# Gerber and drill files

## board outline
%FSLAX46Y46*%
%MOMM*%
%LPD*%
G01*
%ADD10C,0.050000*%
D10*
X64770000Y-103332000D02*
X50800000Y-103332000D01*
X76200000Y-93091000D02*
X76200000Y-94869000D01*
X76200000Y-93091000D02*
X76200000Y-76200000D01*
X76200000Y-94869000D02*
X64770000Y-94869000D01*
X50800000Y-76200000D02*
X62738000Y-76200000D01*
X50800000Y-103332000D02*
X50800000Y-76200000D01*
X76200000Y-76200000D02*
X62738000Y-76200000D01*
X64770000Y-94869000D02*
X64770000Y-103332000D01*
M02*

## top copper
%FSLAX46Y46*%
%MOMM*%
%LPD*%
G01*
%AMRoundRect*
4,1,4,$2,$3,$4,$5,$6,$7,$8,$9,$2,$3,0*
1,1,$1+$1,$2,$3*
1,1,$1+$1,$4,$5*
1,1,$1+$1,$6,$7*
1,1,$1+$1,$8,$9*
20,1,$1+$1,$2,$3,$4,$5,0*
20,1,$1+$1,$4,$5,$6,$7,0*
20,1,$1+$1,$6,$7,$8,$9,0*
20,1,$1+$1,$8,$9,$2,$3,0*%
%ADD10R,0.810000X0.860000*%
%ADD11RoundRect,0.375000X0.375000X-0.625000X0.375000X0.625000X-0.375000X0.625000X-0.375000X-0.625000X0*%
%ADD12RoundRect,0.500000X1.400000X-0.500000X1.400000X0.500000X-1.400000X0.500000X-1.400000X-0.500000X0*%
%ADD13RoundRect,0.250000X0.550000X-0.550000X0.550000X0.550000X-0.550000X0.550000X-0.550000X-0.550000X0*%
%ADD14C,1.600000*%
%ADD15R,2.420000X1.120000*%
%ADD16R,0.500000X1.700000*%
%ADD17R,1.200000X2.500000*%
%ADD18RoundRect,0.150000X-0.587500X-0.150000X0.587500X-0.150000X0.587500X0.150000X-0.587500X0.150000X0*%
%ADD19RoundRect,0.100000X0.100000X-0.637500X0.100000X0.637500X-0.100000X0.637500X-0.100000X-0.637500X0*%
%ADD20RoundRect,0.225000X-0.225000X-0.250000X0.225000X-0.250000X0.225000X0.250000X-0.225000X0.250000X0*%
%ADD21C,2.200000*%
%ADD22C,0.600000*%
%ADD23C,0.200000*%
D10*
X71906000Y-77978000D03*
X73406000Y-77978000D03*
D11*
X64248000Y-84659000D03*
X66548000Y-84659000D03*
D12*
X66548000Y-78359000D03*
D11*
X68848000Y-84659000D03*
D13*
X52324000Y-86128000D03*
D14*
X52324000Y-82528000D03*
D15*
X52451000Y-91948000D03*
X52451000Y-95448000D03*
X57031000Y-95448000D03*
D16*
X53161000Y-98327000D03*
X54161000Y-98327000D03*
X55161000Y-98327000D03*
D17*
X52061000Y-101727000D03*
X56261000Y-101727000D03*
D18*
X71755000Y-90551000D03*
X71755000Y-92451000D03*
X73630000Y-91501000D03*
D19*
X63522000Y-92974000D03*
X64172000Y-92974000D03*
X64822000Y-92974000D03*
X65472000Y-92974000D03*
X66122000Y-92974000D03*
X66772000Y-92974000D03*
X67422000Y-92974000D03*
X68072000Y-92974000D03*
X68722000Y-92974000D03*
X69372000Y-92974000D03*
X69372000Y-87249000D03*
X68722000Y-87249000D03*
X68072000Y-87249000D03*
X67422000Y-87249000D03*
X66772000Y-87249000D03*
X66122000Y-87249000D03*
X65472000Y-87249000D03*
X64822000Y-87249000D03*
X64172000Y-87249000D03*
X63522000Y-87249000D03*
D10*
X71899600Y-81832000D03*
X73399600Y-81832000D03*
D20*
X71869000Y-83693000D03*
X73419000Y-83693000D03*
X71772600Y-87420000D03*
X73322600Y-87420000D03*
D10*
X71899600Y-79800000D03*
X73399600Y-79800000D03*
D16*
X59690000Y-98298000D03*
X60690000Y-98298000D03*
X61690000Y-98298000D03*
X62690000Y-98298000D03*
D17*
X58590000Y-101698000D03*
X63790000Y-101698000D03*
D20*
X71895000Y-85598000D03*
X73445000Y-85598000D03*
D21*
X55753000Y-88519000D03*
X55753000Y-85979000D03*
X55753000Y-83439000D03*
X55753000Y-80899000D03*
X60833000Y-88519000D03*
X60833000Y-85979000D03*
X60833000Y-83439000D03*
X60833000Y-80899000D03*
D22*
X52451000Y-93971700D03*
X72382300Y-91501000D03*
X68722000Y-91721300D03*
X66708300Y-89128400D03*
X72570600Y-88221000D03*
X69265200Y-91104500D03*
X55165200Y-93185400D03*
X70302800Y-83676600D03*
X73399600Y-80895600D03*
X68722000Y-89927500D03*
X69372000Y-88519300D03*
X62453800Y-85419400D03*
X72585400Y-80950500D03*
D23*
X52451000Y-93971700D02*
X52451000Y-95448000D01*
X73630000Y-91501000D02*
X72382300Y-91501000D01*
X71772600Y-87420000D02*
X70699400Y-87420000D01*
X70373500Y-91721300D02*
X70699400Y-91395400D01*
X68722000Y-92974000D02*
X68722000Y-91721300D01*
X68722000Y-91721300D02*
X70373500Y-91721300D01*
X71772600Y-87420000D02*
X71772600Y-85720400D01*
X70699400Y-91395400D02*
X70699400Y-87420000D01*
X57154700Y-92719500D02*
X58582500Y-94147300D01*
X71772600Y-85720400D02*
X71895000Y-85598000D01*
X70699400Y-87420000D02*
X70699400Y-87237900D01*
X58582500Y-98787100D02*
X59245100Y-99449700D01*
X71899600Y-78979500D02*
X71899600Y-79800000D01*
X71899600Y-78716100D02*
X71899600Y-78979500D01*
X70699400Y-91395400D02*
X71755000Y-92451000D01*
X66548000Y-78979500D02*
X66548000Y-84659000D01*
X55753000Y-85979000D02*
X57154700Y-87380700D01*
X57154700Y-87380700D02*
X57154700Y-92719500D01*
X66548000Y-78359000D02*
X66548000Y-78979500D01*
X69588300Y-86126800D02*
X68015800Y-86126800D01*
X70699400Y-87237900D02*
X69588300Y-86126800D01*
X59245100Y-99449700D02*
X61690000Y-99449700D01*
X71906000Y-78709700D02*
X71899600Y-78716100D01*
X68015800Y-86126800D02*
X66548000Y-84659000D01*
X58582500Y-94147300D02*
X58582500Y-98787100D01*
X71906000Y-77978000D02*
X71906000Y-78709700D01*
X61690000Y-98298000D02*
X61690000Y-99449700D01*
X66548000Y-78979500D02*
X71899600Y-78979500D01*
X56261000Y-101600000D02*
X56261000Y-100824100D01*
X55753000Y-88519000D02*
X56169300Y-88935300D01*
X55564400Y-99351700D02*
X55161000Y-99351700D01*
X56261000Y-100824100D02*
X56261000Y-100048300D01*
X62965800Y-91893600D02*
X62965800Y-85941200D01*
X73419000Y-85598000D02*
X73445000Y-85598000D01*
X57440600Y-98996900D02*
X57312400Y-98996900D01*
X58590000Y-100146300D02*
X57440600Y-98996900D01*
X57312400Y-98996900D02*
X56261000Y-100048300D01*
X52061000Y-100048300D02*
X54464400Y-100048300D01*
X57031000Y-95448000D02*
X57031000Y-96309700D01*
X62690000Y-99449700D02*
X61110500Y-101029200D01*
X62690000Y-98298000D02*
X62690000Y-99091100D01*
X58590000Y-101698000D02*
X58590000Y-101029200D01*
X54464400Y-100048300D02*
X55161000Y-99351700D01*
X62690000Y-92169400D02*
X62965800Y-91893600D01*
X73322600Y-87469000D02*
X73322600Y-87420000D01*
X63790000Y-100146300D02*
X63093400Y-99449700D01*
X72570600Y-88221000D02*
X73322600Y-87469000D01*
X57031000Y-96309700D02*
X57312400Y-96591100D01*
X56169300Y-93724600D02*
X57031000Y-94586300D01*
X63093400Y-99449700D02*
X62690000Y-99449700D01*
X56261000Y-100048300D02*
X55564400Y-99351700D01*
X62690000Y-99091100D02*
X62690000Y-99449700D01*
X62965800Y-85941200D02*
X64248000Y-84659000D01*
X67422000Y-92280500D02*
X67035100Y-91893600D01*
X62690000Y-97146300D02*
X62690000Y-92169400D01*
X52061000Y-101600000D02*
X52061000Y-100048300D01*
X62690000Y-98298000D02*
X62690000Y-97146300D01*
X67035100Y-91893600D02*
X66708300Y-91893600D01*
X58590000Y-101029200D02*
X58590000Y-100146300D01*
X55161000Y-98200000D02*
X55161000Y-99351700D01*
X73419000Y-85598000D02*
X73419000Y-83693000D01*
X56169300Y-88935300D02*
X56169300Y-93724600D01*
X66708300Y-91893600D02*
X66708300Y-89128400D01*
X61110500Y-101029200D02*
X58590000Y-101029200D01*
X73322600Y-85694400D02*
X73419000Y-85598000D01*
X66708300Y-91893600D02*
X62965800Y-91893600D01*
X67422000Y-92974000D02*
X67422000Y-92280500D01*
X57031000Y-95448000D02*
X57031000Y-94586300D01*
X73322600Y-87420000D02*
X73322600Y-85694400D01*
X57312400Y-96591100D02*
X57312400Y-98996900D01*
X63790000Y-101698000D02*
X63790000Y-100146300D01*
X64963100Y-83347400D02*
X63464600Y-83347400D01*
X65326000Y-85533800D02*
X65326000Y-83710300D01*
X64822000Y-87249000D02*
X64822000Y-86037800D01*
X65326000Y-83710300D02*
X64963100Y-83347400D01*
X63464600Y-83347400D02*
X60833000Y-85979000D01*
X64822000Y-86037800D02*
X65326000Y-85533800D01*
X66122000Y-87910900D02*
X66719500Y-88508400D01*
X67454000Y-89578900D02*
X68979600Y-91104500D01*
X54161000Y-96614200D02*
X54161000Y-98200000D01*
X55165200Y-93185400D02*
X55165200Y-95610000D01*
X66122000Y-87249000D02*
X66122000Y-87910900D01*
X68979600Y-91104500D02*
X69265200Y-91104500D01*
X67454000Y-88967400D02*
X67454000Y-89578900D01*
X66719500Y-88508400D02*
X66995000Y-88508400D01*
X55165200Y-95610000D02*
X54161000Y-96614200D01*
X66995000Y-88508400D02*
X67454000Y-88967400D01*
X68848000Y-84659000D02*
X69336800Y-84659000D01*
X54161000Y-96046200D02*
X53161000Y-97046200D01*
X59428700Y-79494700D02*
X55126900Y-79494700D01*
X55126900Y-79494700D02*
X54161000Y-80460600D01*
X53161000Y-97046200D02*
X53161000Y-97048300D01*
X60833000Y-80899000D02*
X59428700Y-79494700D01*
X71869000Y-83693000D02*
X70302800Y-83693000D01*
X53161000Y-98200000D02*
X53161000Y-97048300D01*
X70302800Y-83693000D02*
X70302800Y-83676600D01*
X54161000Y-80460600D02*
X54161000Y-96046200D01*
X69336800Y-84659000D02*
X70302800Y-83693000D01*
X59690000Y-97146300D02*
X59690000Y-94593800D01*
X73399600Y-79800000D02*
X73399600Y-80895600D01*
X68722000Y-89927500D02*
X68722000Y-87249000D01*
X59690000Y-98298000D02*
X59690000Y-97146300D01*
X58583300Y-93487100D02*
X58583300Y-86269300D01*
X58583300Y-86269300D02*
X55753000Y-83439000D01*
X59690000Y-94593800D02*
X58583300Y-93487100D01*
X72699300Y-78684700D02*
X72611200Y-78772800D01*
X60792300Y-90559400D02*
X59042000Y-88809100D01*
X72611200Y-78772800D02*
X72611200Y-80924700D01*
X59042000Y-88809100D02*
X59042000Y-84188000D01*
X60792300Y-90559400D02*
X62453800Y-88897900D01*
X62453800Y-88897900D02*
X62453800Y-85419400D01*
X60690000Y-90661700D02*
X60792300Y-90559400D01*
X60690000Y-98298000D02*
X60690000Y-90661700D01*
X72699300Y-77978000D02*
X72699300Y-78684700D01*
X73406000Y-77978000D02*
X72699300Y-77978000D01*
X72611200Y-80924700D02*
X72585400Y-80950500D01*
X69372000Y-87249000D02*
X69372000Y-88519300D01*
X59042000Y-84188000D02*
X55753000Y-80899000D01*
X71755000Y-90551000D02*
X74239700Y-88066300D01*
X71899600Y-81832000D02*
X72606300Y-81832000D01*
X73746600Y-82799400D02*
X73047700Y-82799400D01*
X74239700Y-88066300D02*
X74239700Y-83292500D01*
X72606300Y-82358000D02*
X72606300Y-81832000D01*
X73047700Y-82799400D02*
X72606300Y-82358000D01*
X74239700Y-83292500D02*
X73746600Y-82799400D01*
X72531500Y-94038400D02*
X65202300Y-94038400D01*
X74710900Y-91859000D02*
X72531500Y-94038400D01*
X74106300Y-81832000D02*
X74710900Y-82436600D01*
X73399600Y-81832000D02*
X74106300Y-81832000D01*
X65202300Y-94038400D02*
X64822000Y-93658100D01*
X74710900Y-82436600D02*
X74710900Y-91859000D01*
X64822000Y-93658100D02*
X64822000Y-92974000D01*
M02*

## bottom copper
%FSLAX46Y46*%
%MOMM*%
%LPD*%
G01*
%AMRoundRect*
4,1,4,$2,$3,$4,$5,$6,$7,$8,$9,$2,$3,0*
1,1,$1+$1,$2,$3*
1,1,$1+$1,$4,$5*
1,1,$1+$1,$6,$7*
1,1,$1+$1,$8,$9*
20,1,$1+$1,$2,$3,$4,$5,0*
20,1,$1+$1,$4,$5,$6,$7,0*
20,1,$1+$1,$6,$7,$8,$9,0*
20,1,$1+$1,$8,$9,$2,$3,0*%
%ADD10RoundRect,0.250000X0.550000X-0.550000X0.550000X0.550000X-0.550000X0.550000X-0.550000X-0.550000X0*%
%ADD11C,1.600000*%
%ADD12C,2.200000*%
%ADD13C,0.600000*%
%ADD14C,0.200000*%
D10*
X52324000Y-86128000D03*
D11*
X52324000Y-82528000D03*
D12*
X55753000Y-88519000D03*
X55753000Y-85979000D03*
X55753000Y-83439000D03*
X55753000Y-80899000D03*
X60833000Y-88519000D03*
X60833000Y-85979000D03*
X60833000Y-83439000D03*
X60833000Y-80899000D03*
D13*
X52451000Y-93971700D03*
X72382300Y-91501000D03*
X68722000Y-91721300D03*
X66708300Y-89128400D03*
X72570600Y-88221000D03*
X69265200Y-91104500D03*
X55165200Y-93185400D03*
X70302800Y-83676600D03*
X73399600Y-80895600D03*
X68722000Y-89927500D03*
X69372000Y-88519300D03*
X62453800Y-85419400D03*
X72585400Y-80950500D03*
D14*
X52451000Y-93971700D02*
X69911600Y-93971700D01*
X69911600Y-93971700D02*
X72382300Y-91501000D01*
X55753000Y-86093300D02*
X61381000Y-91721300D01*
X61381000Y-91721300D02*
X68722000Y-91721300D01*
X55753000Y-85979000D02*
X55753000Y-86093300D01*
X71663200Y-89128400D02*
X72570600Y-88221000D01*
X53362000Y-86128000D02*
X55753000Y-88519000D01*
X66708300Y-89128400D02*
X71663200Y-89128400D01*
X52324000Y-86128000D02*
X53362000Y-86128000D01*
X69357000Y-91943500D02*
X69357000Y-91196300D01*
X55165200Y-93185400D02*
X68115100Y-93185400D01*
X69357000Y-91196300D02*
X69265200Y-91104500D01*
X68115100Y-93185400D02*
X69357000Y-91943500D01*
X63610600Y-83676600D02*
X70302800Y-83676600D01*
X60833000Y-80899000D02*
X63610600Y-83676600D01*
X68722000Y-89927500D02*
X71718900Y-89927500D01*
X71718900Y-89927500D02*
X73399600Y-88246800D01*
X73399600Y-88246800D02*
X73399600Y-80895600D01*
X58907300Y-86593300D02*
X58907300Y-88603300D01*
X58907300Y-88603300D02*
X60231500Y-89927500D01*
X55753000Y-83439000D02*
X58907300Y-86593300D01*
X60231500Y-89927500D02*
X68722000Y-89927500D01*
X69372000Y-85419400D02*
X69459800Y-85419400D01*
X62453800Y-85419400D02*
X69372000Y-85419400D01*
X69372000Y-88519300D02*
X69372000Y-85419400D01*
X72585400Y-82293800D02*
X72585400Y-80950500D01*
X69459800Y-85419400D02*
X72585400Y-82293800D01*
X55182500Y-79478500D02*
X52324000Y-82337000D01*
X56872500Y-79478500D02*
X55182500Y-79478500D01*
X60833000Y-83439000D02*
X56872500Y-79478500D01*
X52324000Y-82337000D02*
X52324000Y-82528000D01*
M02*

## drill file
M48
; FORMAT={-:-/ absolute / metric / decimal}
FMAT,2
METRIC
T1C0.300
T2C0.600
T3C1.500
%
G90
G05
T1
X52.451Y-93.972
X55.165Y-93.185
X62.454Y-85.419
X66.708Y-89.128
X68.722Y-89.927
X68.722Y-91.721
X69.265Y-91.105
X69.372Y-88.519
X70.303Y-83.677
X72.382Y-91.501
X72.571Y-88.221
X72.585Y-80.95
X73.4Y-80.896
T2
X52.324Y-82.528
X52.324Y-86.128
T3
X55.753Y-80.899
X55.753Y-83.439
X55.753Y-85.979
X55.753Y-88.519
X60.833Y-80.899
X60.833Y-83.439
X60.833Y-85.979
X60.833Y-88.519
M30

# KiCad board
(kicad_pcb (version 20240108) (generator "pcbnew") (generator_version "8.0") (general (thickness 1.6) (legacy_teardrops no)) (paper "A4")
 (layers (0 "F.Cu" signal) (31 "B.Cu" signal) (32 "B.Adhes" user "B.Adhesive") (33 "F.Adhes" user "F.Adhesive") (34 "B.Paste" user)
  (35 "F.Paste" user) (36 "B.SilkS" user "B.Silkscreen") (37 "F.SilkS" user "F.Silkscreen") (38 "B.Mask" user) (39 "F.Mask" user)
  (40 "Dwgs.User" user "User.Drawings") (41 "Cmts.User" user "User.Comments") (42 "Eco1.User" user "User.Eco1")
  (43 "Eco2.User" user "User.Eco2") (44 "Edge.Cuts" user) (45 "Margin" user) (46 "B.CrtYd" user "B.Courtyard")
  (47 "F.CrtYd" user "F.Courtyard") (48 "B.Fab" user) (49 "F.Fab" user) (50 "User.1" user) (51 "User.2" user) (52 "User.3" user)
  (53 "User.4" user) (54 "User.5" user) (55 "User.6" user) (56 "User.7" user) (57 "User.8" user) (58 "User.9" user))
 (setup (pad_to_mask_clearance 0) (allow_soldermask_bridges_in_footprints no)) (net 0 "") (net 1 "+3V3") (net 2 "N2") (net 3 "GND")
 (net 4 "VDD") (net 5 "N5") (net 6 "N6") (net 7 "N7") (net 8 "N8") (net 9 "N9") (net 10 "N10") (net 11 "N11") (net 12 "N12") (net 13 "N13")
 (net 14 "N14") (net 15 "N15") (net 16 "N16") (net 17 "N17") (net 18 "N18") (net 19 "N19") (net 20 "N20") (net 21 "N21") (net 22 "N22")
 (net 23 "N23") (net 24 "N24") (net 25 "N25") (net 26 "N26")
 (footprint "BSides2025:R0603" (layer "F.Cu") (at 72.656 77.978)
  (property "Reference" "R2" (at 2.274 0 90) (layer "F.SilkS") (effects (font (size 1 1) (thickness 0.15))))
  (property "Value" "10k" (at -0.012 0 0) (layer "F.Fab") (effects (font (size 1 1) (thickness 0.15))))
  (pad "1" smd rect (at -0.75 0) (size 0.81 0.86) (layers "F.Cu" "F.Paste" "F.Mask") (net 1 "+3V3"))
  (pad "2" smd rect (at 0.75 0) (size 0.81 0.86) (layers "F.Cu" "F.Paste" "F.Mask") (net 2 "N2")))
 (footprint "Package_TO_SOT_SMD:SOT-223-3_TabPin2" (layer "F.Cu") (at 66.548 81.509 90)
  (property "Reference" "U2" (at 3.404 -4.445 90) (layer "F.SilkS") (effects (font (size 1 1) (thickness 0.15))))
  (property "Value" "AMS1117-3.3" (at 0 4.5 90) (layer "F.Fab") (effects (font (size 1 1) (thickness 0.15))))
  (pad "1" smd roundrect (at -3.15 -2.3 90) (size 2 1.5) (layers "F.Cu" "F.Paste" "F.Mask") (roundrect_rratio 0.25) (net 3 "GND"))
  (pad "2" smd roundrect (at -3.15 0 90) (size 2 1.5) (layers "F.Cu" "F.Paste" "F.Mask") (roundrect_rratio 0.25) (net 1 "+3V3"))
  (pad "2" smd roundrect (at 3.15 0 90) (size 2 3.8) (layers "F.Cu" "F.Paste" "F.Mask") (roundrect_rratio 0.25) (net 1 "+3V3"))
  (pad "3" smd roundrect (at -3.15 2.3 90) (size 2 1.5) (layers "F.Cu" "F.Paste" "F.Mask") (roundrect_rratio 0.25) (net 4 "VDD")))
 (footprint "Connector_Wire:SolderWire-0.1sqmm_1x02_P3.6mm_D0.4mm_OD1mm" (layer "F.Cu") (at 52.324 86.128 90)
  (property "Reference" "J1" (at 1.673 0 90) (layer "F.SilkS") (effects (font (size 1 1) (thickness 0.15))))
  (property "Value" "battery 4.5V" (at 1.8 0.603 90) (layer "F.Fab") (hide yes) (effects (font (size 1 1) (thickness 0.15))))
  (pad "1" thru_hole roundrect (at 0 0 90) (size 1.6 1.6) (drill 0.6) (layers "*.Cu" "*.Mask") (remove_unused_layers no)
   (roundrect_rratio 0.15625) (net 3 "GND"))
  (pad "2" thru_hole circle (at 3.6 0 90) (size 1.6 1.6) (drill 0.6) (layers "*.Cu" "*.Mask") (remove_unused_layers no) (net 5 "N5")))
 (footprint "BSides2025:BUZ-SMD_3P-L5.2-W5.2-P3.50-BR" (layer "F.Cu") (at 54.741 93.698 90)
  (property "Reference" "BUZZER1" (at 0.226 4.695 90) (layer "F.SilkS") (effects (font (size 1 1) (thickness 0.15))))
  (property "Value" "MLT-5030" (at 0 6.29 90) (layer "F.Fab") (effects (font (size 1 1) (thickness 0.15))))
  (pad "1" smd rect (at 1.75 -2.29 270) (size 1.12 2.42) (layers "F.Cu" "F.Paste" "F.Mask") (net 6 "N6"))
  (pad "2" smd rect (at -1.75 -2.29 270) (size 1.12 2.42) (layers "F.Cu" "F.Paste" "F.Mask") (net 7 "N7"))
  (pad "3" smd rect (at -1.75 2.29 270) (size 1.12 2.42) (layers "F.Cu" "F.Paste" "F.Mask") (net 3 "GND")))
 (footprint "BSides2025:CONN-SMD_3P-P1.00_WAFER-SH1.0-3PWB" (layer "F.Cu") (at 54.161 100.027)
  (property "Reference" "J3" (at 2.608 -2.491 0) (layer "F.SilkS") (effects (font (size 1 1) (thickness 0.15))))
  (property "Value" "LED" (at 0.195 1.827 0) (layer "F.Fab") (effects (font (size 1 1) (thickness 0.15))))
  (pad "1" smd rect (at -1 -1.7) (size 0.5 1.7) (layers "F.Cu" "F.Paste" "F.Mask") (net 4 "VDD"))
  (pad "2" smd rect (at 0 -1.7) (size 0.5 1.7) (layers "F.Cu" "F.Paste" "F.Mask") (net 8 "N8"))
  (pad "3" smd rect (at 1 -1.7) (size 0.5 1.7) (layers "F.Cu" "F.Paste" "F.Mask") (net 3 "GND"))
  (pad "4" smd rect (at -2.1 1.7) (size 1.2 2.5) (layers "F.Cu" "F.Paste" "F.Mask") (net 3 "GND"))
  (pad "5" smd rect (at 2.1 1.7) (size 1.2 2.5) (layers "F.Cu" "F.Paste" "F.Mask") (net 3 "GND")))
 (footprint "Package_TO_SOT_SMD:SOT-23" (layer "F.Cu") (at 72.6925 91.501)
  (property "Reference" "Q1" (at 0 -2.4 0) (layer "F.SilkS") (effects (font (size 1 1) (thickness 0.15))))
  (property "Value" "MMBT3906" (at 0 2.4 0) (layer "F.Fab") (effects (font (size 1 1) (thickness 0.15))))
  (pad "1" smd roundrect (at -0.9375 -0.95) (size 1.475 0.6) (layers "F.Cu" "F.Paste" "F.Mask") (roundrect_rratio 0.25) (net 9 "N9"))
  (pad "2" smd roundrect (at -0.9375 0.95) (size 1.475 0.6) (layers "F.Cu" "F.Paste" "F.Mask") (roundrect_rratio 0.25) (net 1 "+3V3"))
  (pad "3" smd roundrect (at 0.9375 0) (size 1.475 0.6) (layers "F.Cu" "F.Paste" "F.Mask") (roundrect_rratio 0.25) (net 7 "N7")))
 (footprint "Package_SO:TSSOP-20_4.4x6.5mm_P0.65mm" (layer "F.Cu") (at 66.447 90.1115 90)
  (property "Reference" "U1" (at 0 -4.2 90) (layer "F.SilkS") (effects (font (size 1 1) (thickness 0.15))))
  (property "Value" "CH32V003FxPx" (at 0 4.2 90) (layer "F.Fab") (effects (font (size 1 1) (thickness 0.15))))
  (pad "1" smd roundrect (at -2.8625 -2.925 90) (size 1.475 0.4) (layers "F.Cu" "F.Paste" "F.Mask") (roundrect_rratio 0.25) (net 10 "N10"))
  (pad "2" smd roundrect (at -2.8625 -2.275 90) (size 1.475 0.4) (layers "F.Cu" "F.Paste" "F.Mask") (roundrect_rratio 0.25) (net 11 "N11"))
  (pad "3" smd roundrect (at -2.8625 -1.625 90) (size 1.475 0.4) (layers "F.Cu" "F.Paste" "F.Mask") (roundrect_rratio 0.25) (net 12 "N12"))
  (pad "4" smd roundrect (at -2.8625 -0.975 90) (size 1.475 0.4) (layers "F.Cu" "F.Paste" "F.Mask") (roundrect_rratio 0.25) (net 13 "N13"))
  (pad "5" smd roundrect (at -2.8625 -0.325 90) (size 1.475 0.4) (layers "F.Cu" "F.Paste" "F.Mask") (roundrect_rratio 0.25) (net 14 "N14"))
  (pad "6" smd roundrect (at -2.8625 0.325 90) (size 1.475 0.4) (layers "F.Cu" "F.Paste" "F.Mask") (roundrect_rratio 0.25) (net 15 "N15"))
  (pad "7" smd roundrect (at -2.8625 0.975 90) (size 1.475 0.4) (layers "F.Cu" "F.Paste" "F.Mask") (roundrect_rratio 0.25) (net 3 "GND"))
  (pad "8" smd roundrect (at -2.8625 1.625 90) (size 1.475 0.4) (layers "F.Cu" "F.Paste" "F.Mask") (roundrect_rratio 0.25) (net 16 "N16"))
  (pad "9" smd roundrect (at -2.8625 2.275 90) (size 1.475 0.4) (layers "F.Cu" "F.Paste" "F.Mask") (roundrect_rratio 0.25) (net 1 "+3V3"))
  (pad "10" smd roundrect (at -2.8625 2.925 90) (size 1.475 0.4) (layers "F.Cu" "F.Paste" "F.Mask") (roundrect_rratio 0.25) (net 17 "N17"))
  (pad "11" smd roundrect (at 2.8625 2.925 90) (size 1.475 0.4) (layers "F.Cu" "F.Paste" "F.Mask") (roundrect_rratio 0.25) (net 2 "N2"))
  (pad "12" smd roundrect (at 2.8625 2.275 90) (size 1.475 0.4) (layers "F.Cu" "F.Paste" "F.Mask") (roundrect_rratio 0.25) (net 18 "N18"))
  (pad "13" smd roundrect (at 2.8625 1.625 90) (size 1.475 0.4) (layers "F.Cu" "F.Paste" "F.Mask") (roundrect_rratio 0.25) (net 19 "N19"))
  (pad "14" smd roundrect (at 2.8625 0.975 90) (size 1.475 0.4) (layers "F.Cu" "F.Paste" "F.Mask") (roundrect_rratio 0.25) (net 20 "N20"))
  (pad "15" smd roundrect (at 2.8625 0.325 90) (size 1.475 0.4) (layers "F.Cu" "F.Paste" "F.Mask") (roundrect_rratio 0.25) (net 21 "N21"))
  (pad "16" smd roundrect (at 2.8625 -0.325 90) (size 1.475 0.4) (layers "F.Cu" "F.Paste" "F.Mask") (roundrect_rratio 0.25) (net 8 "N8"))
  (pad "17" smd roundrect (at 2.8625 -0.975 90) (size 1.475 0.4) (layers "F.Cu" "F.Paste" "F.Mask") (roundrect_rratio 0.25) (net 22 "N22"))
  (pad "18" smd roundrect (at 2.8625 -1.625 90) (size 1.475 0.4) (layers "F.Cu" "F.Paste" "F.Mask") (roundrect_rratio 0.25) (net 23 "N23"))
  (pad "19" smd roundrect (at 2.8625 -2.275 90) (size 1.475 0.4) (layers "F.Cu" "F.Paste" "F.Mask") (roundrect_rratio 0.25) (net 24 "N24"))
  (pad "20" smd roundrect (at 2.8625 -2.925 90) (size 1.475 0.4) (layers "F.Cu" "F.Paste" "F.Mask") (roundrect_rratio 0.25) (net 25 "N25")))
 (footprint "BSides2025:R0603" (layer "F.Cu") (at 72.6496 81.832)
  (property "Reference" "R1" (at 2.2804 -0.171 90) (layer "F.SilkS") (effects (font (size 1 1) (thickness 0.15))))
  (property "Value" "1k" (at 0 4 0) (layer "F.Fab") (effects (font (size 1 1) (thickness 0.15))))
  (pad "1" smd rect (at -0.75 0) (size 0.81 0.86) (layers "F.Cu" "F.Paste" "F.Mask") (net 9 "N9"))
  (pad "2" smd rect (at 0.75 0) (size 0.81 0.86) (layers "F.Cu" "F.Paste" "F.Mask") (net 12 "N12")))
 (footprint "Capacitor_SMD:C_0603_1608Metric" (layer "F.Cu") (at 72.644 83.693)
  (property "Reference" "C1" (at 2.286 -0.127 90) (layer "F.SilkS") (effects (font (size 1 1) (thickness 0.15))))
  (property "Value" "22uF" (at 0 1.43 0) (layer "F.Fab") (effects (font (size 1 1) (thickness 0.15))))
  (pad "1" smd roundrect (at -0.775 0) (size 0.9 0.95) (layers "F.Cu" "F.Paste" "F.Mask") (roundrect_rratio 0.25) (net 4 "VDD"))
  (pad "2" smd roundrect (at 0.775 0) (size 0.9 0.95) (layers "F.Cu" "F.Paste" "F.Mask") (roundrect_rratio 0.25) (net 3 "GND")))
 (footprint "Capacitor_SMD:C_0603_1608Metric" (layer "F.Cu") (at 72.5476 87.42)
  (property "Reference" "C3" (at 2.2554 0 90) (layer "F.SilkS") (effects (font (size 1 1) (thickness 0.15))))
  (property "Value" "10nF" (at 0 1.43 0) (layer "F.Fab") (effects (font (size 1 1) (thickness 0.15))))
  (pad "1" smd roundrect (at -0.775 0) (size 0.9 0.95) (layers "F.Cu" "F.Paste" "F.Mask") (roundrect_rratio 0.25) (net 1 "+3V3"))
  (pad "2" smd roundrect (at 0.775 0) (size 0.9 0.95) (layers "F.Cu" "F.Paste" "F.Mask") (roundrect_rratio 0.25) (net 3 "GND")))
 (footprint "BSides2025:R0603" (layer "F.Cu") (at 72.6496 79.8)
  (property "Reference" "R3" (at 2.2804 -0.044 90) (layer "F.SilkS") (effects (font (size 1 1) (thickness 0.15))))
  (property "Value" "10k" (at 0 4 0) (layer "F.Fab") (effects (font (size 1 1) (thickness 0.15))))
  (pad "1" smd rect (at -0.75 0) (size 0.81 0.86) (layers "F.Cu" "F.Paste" "F.Mask") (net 1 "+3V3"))
  (pad "2" smd rect (at 0.75 0) (size 0.81 0.86) (layers "F.Cu" "F.Paste" "F.Mask") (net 18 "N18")))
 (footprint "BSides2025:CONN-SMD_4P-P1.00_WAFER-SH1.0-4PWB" (layer "F.Cu") (at 61.19 99.998)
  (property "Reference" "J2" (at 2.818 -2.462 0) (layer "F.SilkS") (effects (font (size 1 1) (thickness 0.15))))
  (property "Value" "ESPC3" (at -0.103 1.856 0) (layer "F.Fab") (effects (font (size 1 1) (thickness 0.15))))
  (pad "1" smd rect (at -1.5 -1.7) (size 0.5 1.7) (layers "F.Cu" "F.Paste" "F.Mask") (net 18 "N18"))
  (pad "2" smd rect (at -0.5 -1.7) (size 0.5 1.7) (layers "F.Cu" "F.Paste" "F.Mask") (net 2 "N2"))
  (pad "3" smd rect (at 0.5 -1.7) (size 0.5 1.7) (layers "F.Cu" "F.Paste" "F.Mask") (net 1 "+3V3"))
  (pad "4" smd rect (at 1.5 -1.7) (size 0.5 1.7) (layers "F.Cu" "F.Paste" "F.Mask") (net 3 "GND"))
  (pad "5" smd rect (at -2.6 1.7) (size 1.2 2.5) (layers "F.Cu" "F.Paste" "F.Mask") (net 3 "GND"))
  (pad "6" smd rect (at 2.6 1.7) (size 1.2 2.5) (layers "F.Cu" "F.Paste" "F.Mask") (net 3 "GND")))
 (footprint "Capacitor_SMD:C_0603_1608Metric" (layer "F.Cu") (at 72.67 85.598)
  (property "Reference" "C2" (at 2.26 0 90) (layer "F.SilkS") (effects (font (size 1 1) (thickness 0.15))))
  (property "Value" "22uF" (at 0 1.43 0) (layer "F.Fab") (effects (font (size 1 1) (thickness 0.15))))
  (pad "1" smd roundrect (at -0.775 0) (size 0.9 0.95) (layers "F.Cu" "F.Paste" "F.Mask") (roundrect_rratio 0.25) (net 1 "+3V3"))
  (pad "2" smd roundrect (at 0.775 0) (size 0.9 0.95) (layers "F.Cu" "F.Paste" "F.Mask") (roundrect_rratio 0.25) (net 3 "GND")))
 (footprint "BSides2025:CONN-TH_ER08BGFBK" (layer "B.Cu") (at 58.293 84.709 -90)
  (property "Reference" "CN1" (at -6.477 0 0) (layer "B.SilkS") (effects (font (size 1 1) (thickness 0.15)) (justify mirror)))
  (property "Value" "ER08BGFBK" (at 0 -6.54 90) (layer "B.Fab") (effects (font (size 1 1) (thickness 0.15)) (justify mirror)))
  (pad "A1" thru_hole circle (at 3.81 2.54 90) (size 2.2 2.2) (drill 1.500022) (layers "*.Cu" "*.Mask") (remove_unused_layers no)
   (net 3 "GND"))
  (pad "A2" thru_hole circle (at 1.27 2.54 90) (size 2.2 2.2) (drill 1.500022) (layers "*.Cu" "*.Mask") (remove_unused_layers no)
   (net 1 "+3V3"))
  (pad "A3" thru_hole circle (at -1.27 2.54 90) (size 2.2 2.2) (drill 1.500022) (layers "*.Cu" "*.Mask") (remove_unused_layers no)
   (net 18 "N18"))
  (pad "A4" thru_hole circle (at -3.81 2.54 90) (size 2.2 2.2) (drill 1.500022) (layers "*.Cu" "*.Mask") (remove_unused_layers no)
   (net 2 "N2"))
  (pad "B1" thru_hole circle (at 3.81 -2.54 90) (size 2.2 2.2) (drill 1.500022) (layers "*.Cu" "*.Mask") (remove_unused_layers no)
   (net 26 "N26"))
  (pad "B2" thru_hole circle (at 1.27 -2.54 90) (size 2.2 2.2) (drill 1.500022) (layers "*.Cu" "*.Mask") (remove_unused_layers no)
   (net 23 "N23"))
  (pad "B3" thru_hole circle (at -1.27 -2.54 90) (size 2.2 2.2) (drill 1.500022) (layers "*.Cu" "*.Mask") (remove_unused_layers no)
   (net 5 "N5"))
  (pad "B4" thru_hole circle (at -3.81 -2.54 90) (size 2.2 2.2) (drill 1.500022) (layers "*.Cu" "*.Mask") (remove_unused_layers no)
   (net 4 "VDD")))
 (gr_line (start 64.77 103.332) (end 50.8 103.332) (stroke (width 0.05) (type default)) (layer "Edge.Cuts"))
 (gr_line (start 76.2 93.091) (end 76.2 94.869) (stroke (width 0.05) (type default)) (layer "Edge.Cuts"))
 (gr_line (start 76.2 93.091) (end 76.2 76.2) (stroke (width 0.05) (type default)) (layer "Edge.Cuts"))
 (gr_line (start 76.2 94.869) (end 64.77 94.869) (stroke (width 0.05) (type default)) (layer "Edge.Cuts"))
 (gr_line (start 50.8 76.2) (end 62.738 76.2) (stroke (width 0.05) (type default)) (layer "Edge.Cuts"))
 (gr_line (start 50.8 103.332) (end 50.8 76.2) (stroke (width 0.05) (type default)) (layer "Edge.Cuts"))
 (gr_line (start 76.2 76.2) (end 62.738 76.2) (stroke (width 0.05) (type default)) (layer "Edge.Cuts"))
 (gr_line (start 64.77 94.869) (end 64.77 103.332) (stroke (width 0.05) (type default)) (layer "Edge.Cuts"))
 (segment (start 52.451 93.9717) (end 52.451 95.448) (width 0.2) (layer "F.Cu") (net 7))
 (segment (start 73.63 91.501) (end 72.3823 91.501) (width 0.2) (layer "F.Cu") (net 7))
 (via (at 52.451 93.9717) (size 0.6) (drill 0.3) (layers "F.Cu" "B.Cu") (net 7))
 (via (at 72.3823 91.501) (size 0.6) (drill 0.3) (layers "F.Cu" "B.Cu") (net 7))
 (segment (start 52.451 93.9717) (end 69.9116 93.9717) (width 0.2) (layer "B.Cu") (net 7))
 (segment (start 69.9116 93.9717) (end 72.3823 91.501) (width 0.2) (layer "B.Cu") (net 7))
 (segment (start 71.7726 87.42) (end 70.6994 87.42) (width 0.2) (layer "F.Cu") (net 1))
 (segment (start 70.3735 91.7213) (end 70.6994 91.3954) (width 0.2) (layer "F.Cu") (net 1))
 (segment (start 68.722 92.974) (end 68.722 91.7213) (width 0.2) (layer "F.Cu") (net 1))
 (segment (start 68.722 91.7213) (end 70.3735 91.7213) (width 0.2) (layer "F.Cu") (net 1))
 (segment (start 71.7726 87.42) (end 71.7726 85.7204) (width 0.2) (layer "F.Cu") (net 1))
 (segment (start 70.6994 91.3954) (end 70.6994 87.42) (width 0.2) (layer "F.Cu") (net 1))
 (segment (start 57.1547 92.7195) (end 58.5825 94.1473) (width 0.2) (layer "F.Cu") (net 1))
 (segment (start 71.7726 85.7204) (end 71.895 85.598) (width 0.2) (layer "F.Cu") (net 1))
 (segment (start 70.6994 87.42) (end 70.6994 87.2379) (width 0.2) (layer "F.Cu") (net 1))
 (segment (start 58.5825 98.7871) (end 59.2451 99.4497) (width 0.2) (layer "F.Cu") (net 1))
 (segment (start 71.8996 78.9795) (end 71.8996 79.8) (width 0.2) (layer "F.Cu") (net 1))
 (segment (start 71.8996 78.7161) (end 71.8996 78.9795) (width 0.2) (layer "F.Cu") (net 1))
 (segment (start 70.6994 91.3954) (end 71.755 92.451) (width 0.2) (layer "F.Cu") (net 1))
 (segment (start 66.548 78.9795) (end 66.548 84.659) (width 0.2) (layer "F.Cu") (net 1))
 (segment (start 55.753 85.979) (end 57.1547 87.3807) (width 0.2) (layer "F.Cu") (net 1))
 (segment (start 57.1547 87.3807) (end 57.1547 92.7195) (width 0.2) (layer "F.Cu") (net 1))
 (segment (start 66.548 78.359) (end 66.548 78.9795) (width 0.2) (layer "F.Cu") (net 1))
 (segment (start 69.5883 86.1268) (end 68.0158 86.1268) (width 0.2) (layer "F.Cu") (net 1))
 (segment (start 70.6994 87.2379) (end 69.5883 86.1268) (width 0.2) (layer "F.Cu") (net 1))
 (segment (start 59.2451 99.4497) (end 61.69 99.4497) (width 0.2) (layer "F.Cu") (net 1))
 (segment (start 71.906 78.7097) (end 71.8996 78.7161) (width 0.2) (layer "F.Cu") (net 1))
 (segment (start 68.0158 86.1268) (end 66.548 84.659) (width 0.2) (layer "F.Cu") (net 1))
 (segment (start 58.5825 94.1473) (end 58.5825 98.7871) (width 0.2) (layer "F.Cu") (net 1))
 (segment (start 71.906 77.978) (end 71.906 78.7097) (width 0.2) (layer "F.Cu") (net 1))
 (segment (start 61.69 98.298) (end 61.69 99.4497) (width 0.2) (layer "F.Cu") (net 1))
 (segment (start 66.548 78.9795) (end 71.8996 78.9795) (width 0.2) (layer "F.Cu") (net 1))
 (via (at 68.722 91.7213) (size 0.6) (drill 0.3) (layers "F.Cu" "B.Cu") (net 1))
 (segment (start 55.753 86.0933) (end 61.381 91.7213) (width 0.2) (layer "B.Cu") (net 1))
 (segment (start 61.381 91.7213) (end 68.722 91.7213) (width 0.2) (layer "B.Cu") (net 1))
 (segment (start 55.753 85.979) (end 55.753 86.0933) (width 0.2) (layer "B.Cu") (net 1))
 (segment (start 56.261 101.6) (end 56.261 100.8241) (width 0.2) (layer "F.Cu") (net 3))
 (segment (start 55.753 88.519) (end 56.1693 88.9353) (width 0.2) (layer "F.Cu") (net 3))
 (segment (start 55.5644 99.3517) (end 55.161 99.3517) (width 0.2) (layer "F.Cu") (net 3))
 (segment (start 56.261 100.8241) (end 56.261 100.0483) (width 0.2) (layer "F.Cu") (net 3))
 (segment (start 62.9658 91.8936) (end 62.9658 85.9412) (width 0.2) (layer "F.Cu") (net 3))
 (segment (start 73.419 85.598) (end 73.445 85.598) (width 0.2) (layer "F.Cu") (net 3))
 (segment (start 57.4406 98.9969) (end 57.3124 98.9969) (width 0.2) (layer "F.Cu") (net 3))
 (segment (start 58.59 100.1463) (end 57.4406 98.9969) (width 0.2) (layer "F.Cu") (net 3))
 (segment (start 57.3124 98.9969) (end 56.261 100.0483) (width 0.2) (layer "F.Cu") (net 3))
 (segment (start 52.061 100.0483) (end 54.4644 100.0483) (width 0.2) (layer "F.Cu") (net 3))
 (segment (start 57.031 95.448) (end 57.031 96.3097) (width 0.2) (layer "F.Cu") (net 3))
 (segment (start 62.69 99.4497) (end 61.1105 101.0292) (width 0.2) (layer "F.Cu") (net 3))
 (segment (start 62.69 98.298) (end 62.69 99.0911) (width 0.2) (layer "F.Cu") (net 3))
 (segment (start 58.59 101.698) (end 58.59 101.0292) (width 0.2) (layer "F.Cu") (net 3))
 (segment (start 54.4644 100.0483) (end 55.161 99.3517) (width 0.2) (layer "F.Cu") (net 3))
 (segment (start 62.69 92.1694) (end 62.9658 91.8936) (width 0.2) (layer "F.Cu") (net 3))
 (segment (start 73.3226 87.469) (end 73.3226 87.42) (width 0.2) (layer "F.Cu") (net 3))
 (segment (start 63.79 100.1463) (end 63.0934 99.4497) (width 0.2) (layer "F.Cu") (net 3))
 (segment (start 72.5706 88.221) (end 73.3226 87.469) (width 0.2) (layer "F.Cu") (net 3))
 (segment (start 57.031 96.3097) (end 57.3124 96.5911) (width 0.2) (layer "F.Cu") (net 3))
 (segment (start 56.1693 93.7246) (end 57.031 94.5863) (width 0.2) (layer "F.Cu") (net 3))
 (segment (start 63.0934 99.4497) (end 62.69 99.4497) (width 0.2) (layer "F.Cu") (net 3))
 (segment (start 56.261 100.0483) (end 55.5644 99.3517) (width 0.2) (layer "F.Cu") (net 3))
 (segment (start 62.69 99.0911) (end 62.69 99.4497) (width 0.2) (layer "F.Cu") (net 3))
 (segment (start 62.9658 85.9412) (end 64.248 84.659) (width 0.2) (layer "F.Cu") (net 3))
 (segment (start 67.422 92.2805) (end 67.0351 91.8936) (width 0.2) (layer "F.Cu") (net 3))
 (segment (start 62.69 97.1463) (end 62.69 92.1694) (width 0.2) (layer "F.Cu") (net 3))
 (segment (start 52.061 101.6) (end 52.061 100.0483) (width 0.2) (layer "F.Cu") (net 3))
 (segment (start 62.69 98.298) (end 62.69 97.1463) (width 0.2) (layer "F.Cu") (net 3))
 (segment (start 67.0351 91.8936) (end 66.7083 91.8936) (width 0.2) (layer "F.Cu") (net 3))
 (segment (start 58.59 101.0292) (end 58.59 100.1463) (width 0.2) (layer "F.Cu") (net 3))
 (segment (start 55.161 98.2) (end 55.161 99.3517) (width 0.2) (layer "F.Cu") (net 3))
 (segment (start 73.419 85.598) (end 73.419 83.693) (width 0.2) (layer "F.Cu") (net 3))
 (segment (start 56.1693 88.9353) (end 56.1693 93.7246) (width 0.2) (layer "F.Cu") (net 3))
 (segment (start 66.7083 91.8936) (end 66.7083 89.1284) (width 0.2) (layer "F.Cu") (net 3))
 (segment (start 61.1105 101.0292) (end 58.59 101.0292) (width 0.2) (layer "F.Cu") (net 3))
 (segment (start 73.3226 85.6944) (end 73.419 85.598) (width 0.2) (layer "F.Cu") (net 3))
 (segment (start 66.7083 91.8936) (end 62.9658 91.8936) (width 0.2) (layer "F.Cu") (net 3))
 (segment (start 67.422 92.974) (end 67.422 92.2805) (width 0.2) (layer "F.Cu") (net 3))
 (segment (start 57.031 95.448) (end 57.031 94.5863) (width 0.2) (layer "F.Cu") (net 3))
 (segment (start 73.3226 87.42) (end 73.3226 85.6944) (width 0.2) (layer "F.Cu") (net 3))
 (segment (start 57.3124 96.5911) (end 57.3124 98.9969) (width 0.2) (layer "F.Cu") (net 3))
 (segment (start 63.79 101.698) (end 63.79 100.1463) (width 0.2) (layer "F.Cu") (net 3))
 (via (at 66.7083 89.1284) (size 0.6) (drill 0.3) (layers "F.Cu" "B.Cu") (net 3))
 (via (at 72.5706 88.221) (size 0.6) (drill 0.3) (layers "F.Cu" "B.Cu") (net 3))
 (segment (start 71.6632 89.1284) (end 72.5706 88.221) (width 0.2) (layer "B.Cu") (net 3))
 (segment (start 53.362 86.128) (end 55.753 88.519) (width 0.2) (layer "B.Cu") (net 3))
 (segment (start 66.7083 89.1284) (end 71.6632 89.1284) (width 0.2) (layer "B.Cu") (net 3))
 (segment (start 52.324 86.128) (end 53.362 86.128) (width 0.2) (layer "B.Cu") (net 3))
 (segment (start 64.9631 83.3474) (end 63.4646 83.3474) (width 0.2) (layer "F.Cu") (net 23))
 (segment (start 65.326 85.5338) (end 65.326 83.7103) (width 0.2) (layer "F.Cu") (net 23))
 (segment (start 64.822 87.249) (end 64.822 86.0378) (width 0.2) (layer "F.Cu") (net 23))
 (segment (start 65.326 83.7103) (end 64.9631 83.3474) (width 0.2) (layer "F.Cu") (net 23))
 (segment (start 63.4646 83.3474) (end 60.833 85.979) (width 0.2) (layer "F.Cu") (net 23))
 (segment (start 64.822 86.0378) (end 65.326 85.5338) (width 0.2) (layer "F.Cu") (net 23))
 (segment (start 66.122 87.9109) (end 66.7195 88.5084) (width 0.2) (layer "F.Cu") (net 8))
 (segment (start 67.454 89.5789) (end 68.9796 91.1045) (width 0.2) (layer "F.Cu") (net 8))
 (segment (start 54.161 96.6142) (end 54.161 98.2) (width 0.2) (layer "F.Cu") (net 8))
 (segment (start 55.1652 93.1854) (end 55.1652 95.61) (width 0.2) (layer "F.Cu") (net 8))
 (segment (start 66.122 87.249) (end 66.122 87.9109) (width 0.2) (layer "F.Cu") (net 8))
 (segment (start 68.9796 91.1045) (end 69.2652 91.1045) (width 0.2) (layer "F.Cu") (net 8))
 (segment (start 67.454 88.9674) (end 67.454 89.5789) (width 0.2) (layer "F.Cu") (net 8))
 (segment (start 66.7195 88.5084) (end 66.995 88.5084) (width 0.2) (layer "F.Cu") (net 8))
 (segment (start 55.1652 95.61) (end 54.161 96.6142) (width 0.2) (layer "F.Cu") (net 8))
 (segment (start 66.995 88.5084) (end 67.454 88.9674) (width 0.2) (layer "F.Cu") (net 8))
 (via (at 69.2652 91.1045) (size 0.6) (drill 0.3) (layers "F.Cu" "B.Cu") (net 8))
 (via (at 55.1652 93.1854) (size 0.6) (drill 0.3) (layers "F.Cu" "B.Cu") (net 8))
 (segment (start 69.357 91.9435) (end 69.357 91.1963) (width 0.2) (layer "B.Cu") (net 8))
 (segment (start 55.1652 93.1854) (end 68.1151 93.1854) (width 0.2) (layer "B.Cu") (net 8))
 (segment (start 69.357 91.1963) (end 69.2652 91.1045) (width 0.2) (layer "B.Cu") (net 8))
 (segment (start 68.1151 93.1854) (end 69.357 91.9435) (width 0.2) (layer "B.Cu") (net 8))
 (segment (start 68.848 84.659) (end 69.3368 84.659) (width 0.2) (layer "F.Cu") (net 4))
 (segment (start 54.161 96.0462) (end 53.161 97.0462) (width 0.2) (layer "F.Cu") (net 4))
 (segment (start 59.4287 79.4947) (end 55.1269 79.4947) (width 0.2) (layer "F.Cu") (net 4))
 (segment (start 55.1269 79.4947) (end 54.161 80.4606) (width 0.2) (layer "F.Cu") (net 4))
 (segment (start 53.161 97.0462) (end 53.161 97.0483) (width 0.2) (layer "F.Cu") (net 4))
 (segment (start 60.833 80.899) (end 59.4287 79.4947) (width 0.2) (layer "F.Cu") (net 4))
 (segment (start 71.869 83.693) (end 70.3028 83.693) (width 0.2) (layer "F.Cu") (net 4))
 (segment (start 53.161 98.2) (end 53.161 97.0483) (width 0.2) (layer "F.Cu") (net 4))
 (segment (start 70.3028 83.693) (end 70.3028 83.6766) (width 0.2) (layer "F.Cu") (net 4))
 (segment (start 54.161 80.4606) (end 54.161 96.0462) (width 0.2) (layer "F.Cu") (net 4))
 (segment (start 69.3368 84.659) (end 70.3028 83.693) (width 0.2) (layer "F.Cu") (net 4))
 (via (at 70.3028 83.6766) (size 0.6) (drill 0.3) (layers "F.Cu" "B.Cu") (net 4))
 (segment (start 63.6106 83.6766) (end 70.3028 83.6766) (width 0.2) (layer "B.Cu") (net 4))
 (segment (start 60.833 80.899) (end 63.6106 83.6766) (width 0.2) (layer "B.Cu") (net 4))
 (segment (start 59.69 97.1463) (end 59.69 94.5938) (width 0.2) (layer "F.Cu") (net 18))
 (segment (start 73.3996 79.8) (end 73.3996 80.8956) (width 0.2) (layer "F.Cu") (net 18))
 (segment (start 68.722 89.9275) (end 68.722 87.249) (width 0.2) (layer "F.Cu") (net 18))
 (segment (start 59.69 98.298) (end 59.69 97.1463) (width 0.2) (layer "F.Cu") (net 18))
 (segment (start 58.5833 93.4871) (end 58.5833 86.2693) (width 0.2) (layer "F.Cu") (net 18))
 (segment (start 58.5833 86.2693) (end 55.753 83.439) (width 0.2) (layer "F.Cu") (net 18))
 (segment (start 59.69 94.5938) (end 58.5833 93.4871) (width 0.2) (layer "F.Cu") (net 18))
 (via (at 73.3996 80.8956) (size 0.6) (drill 0.3) (layers "F.Cu" "B.Cu") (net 18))
 (via (at 68.722 89.9275) (size 0.6) (drill 0.3) (layers "F.Cu" "B.Cu") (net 18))
 (segment (start 68.722 89.9275) (end 71.7189 89.9275) (width 0.2) (layer "B.Cu") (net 18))
 (segment (start 71.7189 89.9275) (end 73.3996 88.2468) (width 0.2) (layer "B.Cu") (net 18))
 (segment (start 73.3996 88.2468) (end 73.3996 80.8956) (width 0.2) (layer "B.Cu") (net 18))
 (segment (start 58.9073 86.5933) (end 58.9073 88.6033) (width 0.2) (layer "B.Cu") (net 18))
 (segment (start 58.9073 88.6033) (end 60.2315 89.9275) (width 0.2) (layer "B.Cu") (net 18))
 (segment (start 55.753 83.439) (end 58.9073 86.5933) (width 0.2) (layer "B.Cu") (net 18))
 (segment (start 60.2315 89.9275) (end 68.722 89.9275) (width 0.2) (layer "B.Cu") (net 18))
 (segment (start 72.6993 78.6847) (end 72.6112 78.7728) (width 0.2) (layer "F.Cu") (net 2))
 (segment (start 60.7923 90.5594) (end 59.042 88.8091) (width 0.2) (layer "F.Cu") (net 2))
 (segment (start 72.6112 78.7728) (end 72.6112 80.9247) (width 0.2) (layer "F.Cu") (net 2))
 (segment (start 59.042 88.8091) (end 59.042 84.188) (width 0.2) (layer "F.Cu") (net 2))
 (segment (start 60.7923 90.5594) (end 62.4538 88.8979) (width 0.2) (layer "F.Cu") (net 2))
 (segment (start 62.4538 88.8979) (end 62.4538 85.4194) (width 0.2) (layer "F.Cu") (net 2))
 (segment (start 60.69 90.6617) (end 60.7923 90.5594) (width 0.2) (layer "F.Cu") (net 2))
 (segment (start 60.69 98.298) (end 60.69 90.6617) (width 0.2) (layer "F.Cu") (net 2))
 (segment (start 72.6993 77.978) (end 72.6993 78.6847) (width 0.2) (layer "F.Cu") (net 2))
 (segment (start 73.406 77.978) (end 72.6993 77.978) (width 0.2) (layer "F.Cu") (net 2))
 (segment (start 72.6112 80.9247) (end 72.5854 80.9505) (width 0.2) (layer "F.Cu") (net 2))
 (segment (start 69.372 87.249) (end 69.372 88.5193) (width 0.2) (layer "F.Cu") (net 2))
 (segment (start 59.042 84.188) (end 55.753 80.899) (width 0.2) (layer "F.Cu") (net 2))
 (via (at 69.372 88.5193) (size 0.6) (drill 0.3) (layers "F.Cu" "B.Cu") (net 2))
 (via (at 62.4538 85.4194) (size 0.6) (drill 0.3) (layers "F.Cu" "B.Cu") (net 2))
 (via (at 72.5854 80.9505) (size 0.6) (drill 0.3) (layers "F.Cu" "B.Cu") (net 2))
 (segment (start 69.372 85.4194) (end 69.4598 85.4194) (width 0.2) (layer "B.Cu") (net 2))
 (segment (start 62.4538 85.4194) (end 69.372 85.4194) (width 0.2) (layer "B.Cu") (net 2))
 (segment (start 69.372 88.5193) (end 69.372 85.4194) (width 0.2) (layer "B.Cu") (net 2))
 (segment (start 72.5854 82.2938) (end 72.5854 80.9505) (width 0.2) (layer "B.Cu") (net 2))
 (segment (start 69.4598 85.4194) (end 72.5854 82.2938) (width 0.2) (layer "B.Cu") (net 2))
 (segment (start 55.1825 79.4785) (end 52.324 82.337) (width 0.2) (layer "B.Cu") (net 5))
 (segment (start 56.8725 79.4785) (end 55.1825 79.4785) (width 0.2) (layer "B.Cu") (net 5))
 (segment (start 60.833 83.439) (end 56.8725 79.4785) (width 0.2) (layer "B.Cu") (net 5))
 (segment (start 52.324 82.337) (end 52.324 82.528) (width 0.2) (layer "B.Cu") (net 5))
 (segment (start 71.755 90.551) (end 74.2397 88.0663) (width 0.2) (layer "F.Cu") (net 9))
 (segment (start 71.8996 81.832) (end 72.6063 81.832) (width 0.2) (layer "F.Cu") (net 9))
 (segment (start 73.7466 82.7994) (end 73.0477 82.7994) (width 0.2) (layer "F.Cu") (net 9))
 (segment (start 74.2397 88.0663) (end 74.2397 83.2925) (width 0.2) (layer "F.Cu") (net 9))
 (segment (start 72.6063 82.358) (end 72.6063 81.832) (width 0.2) (layer "F.Cu") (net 9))
 (segment (start 73.0477 82.7994) (end 72.6063 82.358) (width 0.2) (layer "F.Cu") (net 9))
 (segment (start 74.2397 83.2925) (end 73.7466 82.7994) (width 0.2) (layer "F.Cu") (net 9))
 (segment (start 72.5315 94.0384) (end 65.2023 94.0384) (width 0.2) (layer "F.Cu") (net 12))
 (segment (start 74.7109 91.859) (end 72.5315 94.0384) (width 0.2) (layer "F.Cu") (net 12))
 (segment (start 74.1063 81.832) (end 74.7109 82.4366) (width 0.2) (layer "F.Cu") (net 12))
 (segment (start 73.3996 81.832) (end 74.1063 81.832) (width 0.2) (layer "F.Cu") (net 12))
 (segment (start 65.2023 94.0384) (end 64.822 93.6581) (width 0.2) (layer "F.Cu") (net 12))
 (segment (start 74.7109 82.4366) (end 74.7109 91.859) (width 0.2) (layer "F.Cu") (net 12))
 (segment (start 64.822 93.6581) (end 64.822 92.974) (width 0.2) (layer "F.Cu") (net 12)))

